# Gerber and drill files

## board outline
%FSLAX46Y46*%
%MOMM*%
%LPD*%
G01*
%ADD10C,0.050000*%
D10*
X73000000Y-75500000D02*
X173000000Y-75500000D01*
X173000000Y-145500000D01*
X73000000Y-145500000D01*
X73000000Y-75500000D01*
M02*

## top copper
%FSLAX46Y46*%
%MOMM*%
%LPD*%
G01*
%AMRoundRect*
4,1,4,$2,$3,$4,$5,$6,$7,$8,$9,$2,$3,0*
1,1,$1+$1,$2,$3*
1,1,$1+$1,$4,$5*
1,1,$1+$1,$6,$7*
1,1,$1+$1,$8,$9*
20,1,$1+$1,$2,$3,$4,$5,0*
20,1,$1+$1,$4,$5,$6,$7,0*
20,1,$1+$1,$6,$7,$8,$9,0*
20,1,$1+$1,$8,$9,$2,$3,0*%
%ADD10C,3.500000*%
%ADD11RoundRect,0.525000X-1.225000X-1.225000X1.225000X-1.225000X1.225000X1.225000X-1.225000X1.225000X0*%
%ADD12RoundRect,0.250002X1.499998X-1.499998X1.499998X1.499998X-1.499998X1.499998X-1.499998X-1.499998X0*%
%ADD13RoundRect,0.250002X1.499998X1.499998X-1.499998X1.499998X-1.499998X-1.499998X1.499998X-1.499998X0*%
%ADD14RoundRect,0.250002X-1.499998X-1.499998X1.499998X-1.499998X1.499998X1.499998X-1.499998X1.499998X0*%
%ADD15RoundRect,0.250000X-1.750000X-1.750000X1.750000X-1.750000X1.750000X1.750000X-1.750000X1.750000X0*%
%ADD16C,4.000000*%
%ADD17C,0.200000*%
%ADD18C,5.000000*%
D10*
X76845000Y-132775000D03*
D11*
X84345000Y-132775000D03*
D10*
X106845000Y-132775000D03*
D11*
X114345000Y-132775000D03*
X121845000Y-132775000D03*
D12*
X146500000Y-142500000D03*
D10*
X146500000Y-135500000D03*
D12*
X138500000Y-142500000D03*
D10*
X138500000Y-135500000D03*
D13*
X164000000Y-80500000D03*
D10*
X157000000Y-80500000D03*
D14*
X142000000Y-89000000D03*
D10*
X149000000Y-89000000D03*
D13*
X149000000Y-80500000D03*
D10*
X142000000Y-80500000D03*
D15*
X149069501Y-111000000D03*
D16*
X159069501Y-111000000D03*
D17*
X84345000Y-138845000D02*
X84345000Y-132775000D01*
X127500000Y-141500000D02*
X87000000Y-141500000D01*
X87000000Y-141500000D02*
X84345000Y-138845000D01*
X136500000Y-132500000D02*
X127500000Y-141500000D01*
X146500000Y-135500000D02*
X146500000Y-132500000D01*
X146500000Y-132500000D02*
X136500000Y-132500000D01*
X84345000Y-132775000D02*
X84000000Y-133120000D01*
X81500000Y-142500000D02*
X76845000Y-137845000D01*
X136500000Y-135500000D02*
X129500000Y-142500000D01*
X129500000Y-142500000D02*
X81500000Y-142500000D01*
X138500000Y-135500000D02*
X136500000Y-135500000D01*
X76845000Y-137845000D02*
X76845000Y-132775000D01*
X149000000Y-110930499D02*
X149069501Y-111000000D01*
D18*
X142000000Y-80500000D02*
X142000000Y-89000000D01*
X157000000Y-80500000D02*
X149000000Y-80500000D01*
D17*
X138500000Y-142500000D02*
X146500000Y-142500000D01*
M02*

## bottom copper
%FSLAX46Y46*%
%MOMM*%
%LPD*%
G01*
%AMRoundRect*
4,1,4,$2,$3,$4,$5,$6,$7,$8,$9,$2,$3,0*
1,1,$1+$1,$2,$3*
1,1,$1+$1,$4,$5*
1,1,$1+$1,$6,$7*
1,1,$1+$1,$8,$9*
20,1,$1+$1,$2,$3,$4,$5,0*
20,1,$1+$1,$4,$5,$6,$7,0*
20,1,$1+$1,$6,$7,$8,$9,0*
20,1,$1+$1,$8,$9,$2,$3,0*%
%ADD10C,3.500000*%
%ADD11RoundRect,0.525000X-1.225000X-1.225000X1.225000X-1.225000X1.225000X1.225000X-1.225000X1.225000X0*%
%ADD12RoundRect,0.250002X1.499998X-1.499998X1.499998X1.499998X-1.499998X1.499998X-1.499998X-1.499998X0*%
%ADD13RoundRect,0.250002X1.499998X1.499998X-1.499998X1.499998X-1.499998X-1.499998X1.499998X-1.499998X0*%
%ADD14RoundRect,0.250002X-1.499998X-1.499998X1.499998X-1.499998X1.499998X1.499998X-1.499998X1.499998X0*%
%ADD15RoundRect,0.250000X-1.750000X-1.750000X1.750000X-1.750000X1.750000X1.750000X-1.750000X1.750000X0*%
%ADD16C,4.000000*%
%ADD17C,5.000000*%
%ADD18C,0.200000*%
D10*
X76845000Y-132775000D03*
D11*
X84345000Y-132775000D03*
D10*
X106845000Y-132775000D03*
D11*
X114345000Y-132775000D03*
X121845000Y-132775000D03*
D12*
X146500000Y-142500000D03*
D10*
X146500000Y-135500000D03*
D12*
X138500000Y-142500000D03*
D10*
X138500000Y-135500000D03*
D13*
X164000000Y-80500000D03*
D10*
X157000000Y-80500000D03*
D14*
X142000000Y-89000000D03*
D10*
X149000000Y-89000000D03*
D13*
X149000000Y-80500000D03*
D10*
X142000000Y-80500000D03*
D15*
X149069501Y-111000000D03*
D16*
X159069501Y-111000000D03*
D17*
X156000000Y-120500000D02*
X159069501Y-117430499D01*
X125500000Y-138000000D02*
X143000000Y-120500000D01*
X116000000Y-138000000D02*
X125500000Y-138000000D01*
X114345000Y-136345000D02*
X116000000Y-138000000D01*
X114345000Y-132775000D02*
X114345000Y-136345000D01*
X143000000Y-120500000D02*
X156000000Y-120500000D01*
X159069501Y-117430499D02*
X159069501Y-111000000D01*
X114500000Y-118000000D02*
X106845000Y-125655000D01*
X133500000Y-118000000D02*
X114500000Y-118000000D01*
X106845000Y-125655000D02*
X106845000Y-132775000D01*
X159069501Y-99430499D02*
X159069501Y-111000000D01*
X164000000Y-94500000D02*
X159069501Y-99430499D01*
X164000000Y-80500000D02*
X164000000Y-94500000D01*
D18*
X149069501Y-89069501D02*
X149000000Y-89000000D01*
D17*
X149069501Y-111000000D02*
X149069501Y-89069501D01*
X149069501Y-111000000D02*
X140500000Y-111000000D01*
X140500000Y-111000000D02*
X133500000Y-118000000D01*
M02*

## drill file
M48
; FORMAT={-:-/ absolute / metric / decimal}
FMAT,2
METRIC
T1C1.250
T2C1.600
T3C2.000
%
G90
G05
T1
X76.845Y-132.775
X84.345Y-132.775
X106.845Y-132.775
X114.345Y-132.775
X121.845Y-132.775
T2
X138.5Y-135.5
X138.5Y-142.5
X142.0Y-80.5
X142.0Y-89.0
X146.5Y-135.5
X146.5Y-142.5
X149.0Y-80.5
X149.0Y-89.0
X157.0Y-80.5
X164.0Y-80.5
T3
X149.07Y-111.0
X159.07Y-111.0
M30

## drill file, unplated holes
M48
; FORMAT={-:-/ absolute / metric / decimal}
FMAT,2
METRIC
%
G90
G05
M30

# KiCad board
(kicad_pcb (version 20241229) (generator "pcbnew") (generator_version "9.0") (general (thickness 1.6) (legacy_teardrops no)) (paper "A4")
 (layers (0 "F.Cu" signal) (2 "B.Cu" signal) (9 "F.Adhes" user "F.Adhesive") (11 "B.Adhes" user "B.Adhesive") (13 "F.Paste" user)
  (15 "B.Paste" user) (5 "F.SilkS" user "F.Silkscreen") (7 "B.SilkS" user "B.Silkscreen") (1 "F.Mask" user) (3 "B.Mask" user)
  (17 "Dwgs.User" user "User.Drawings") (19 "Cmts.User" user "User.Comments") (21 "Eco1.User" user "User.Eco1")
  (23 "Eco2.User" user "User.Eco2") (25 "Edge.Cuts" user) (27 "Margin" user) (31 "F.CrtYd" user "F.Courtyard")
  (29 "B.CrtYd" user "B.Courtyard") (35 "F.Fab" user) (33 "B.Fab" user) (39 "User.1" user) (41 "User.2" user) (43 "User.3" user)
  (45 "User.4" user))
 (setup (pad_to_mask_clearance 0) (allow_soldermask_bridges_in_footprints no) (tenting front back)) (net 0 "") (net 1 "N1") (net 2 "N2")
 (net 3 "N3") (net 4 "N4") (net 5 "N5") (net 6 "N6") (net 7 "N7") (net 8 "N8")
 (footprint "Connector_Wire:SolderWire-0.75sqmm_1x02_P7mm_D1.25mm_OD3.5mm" (layer "F.Cu") (at 164 80.5 180)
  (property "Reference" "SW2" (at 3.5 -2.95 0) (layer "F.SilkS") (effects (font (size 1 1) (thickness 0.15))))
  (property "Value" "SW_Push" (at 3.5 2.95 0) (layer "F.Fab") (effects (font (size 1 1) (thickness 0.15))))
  (pad "1" thru_hole roundrect (at 0 0 180) (size 3.5 3.5) (drill 1.6) (layers "*.Cu" "*.Mask") (remove_unused_layers no)
   (roundrect_rratio 0.071429) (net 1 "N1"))
  (pad "2" thru_hole circle (at 7 0 180) (size 3.5 3.5) (drill 1.6) (layers "*.Cu" "*.Mask") (remove_unused_layers no) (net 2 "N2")))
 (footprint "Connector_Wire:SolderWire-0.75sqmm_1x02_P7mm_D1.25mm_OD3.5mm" (layer "F.Cu") (at 142 89)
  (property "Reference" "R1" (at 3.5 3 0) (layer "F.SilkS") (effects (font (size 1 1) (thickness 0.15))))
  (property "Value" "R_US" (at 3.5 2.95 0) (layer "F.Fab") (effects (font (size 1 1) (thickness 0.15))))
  (pad "1" thru_hole roundrect (at 0 0) (size 3.5 3.5) (drill 1.6) (layers "*.Cu" "*.Mask") (remove_unused_layers no)
   (roundrect_rratio 0.071429) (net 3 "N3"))
  (pad "2" thru_hole circle (at 7 0) (size 3.5 3.5) (drill 1.6) (layers "*.Cu" "*.Mask") (remove_unused_layers no) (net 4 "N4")))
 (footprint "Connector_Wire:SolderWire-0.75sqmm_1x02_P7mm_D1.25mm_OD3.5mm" (layer "F.Cu") (at 138.5 142.5 90)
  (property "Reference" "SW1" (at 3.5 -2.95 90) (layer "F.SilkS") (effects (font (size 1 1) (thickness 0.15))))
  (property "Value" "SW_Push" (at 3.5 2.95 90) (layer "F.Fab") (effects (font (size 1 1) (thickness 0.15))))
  (pad "1" thru_hole roundrect (at 0 0 90) (size 3.5 3.5) (drill 1.6) (layers "*.Cu" "*.Mask") (remove_unused_layers no)
   (roundrect_rratio 0.071429) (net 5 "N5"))
  (pad "2" thru_hole circle (at 7 0 90) (size 3.5 3.5) (drill 1.6) (layers "*.Cu" "*.Mask") (remove_unused_layers no) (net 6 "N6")))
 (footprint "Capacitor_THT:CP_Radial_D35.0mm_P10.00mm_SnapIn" (layer "F.Cu") (at 149.069501 111)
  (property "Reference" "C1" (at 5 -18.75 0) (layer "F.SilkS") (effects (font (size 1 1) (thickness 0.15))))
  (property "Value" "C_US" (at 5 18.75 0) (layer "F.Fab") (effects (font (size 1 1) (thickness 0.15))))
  (pad "1" thru_hole roundrect (at 0 0) (size 4 4) (drill 2) (layers "*.Cu" "*.Mask") (remove_unused_layers no) (roundrect_rratio 0.0625)
   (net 4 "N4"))
  (pad "2" thru_hole circle (at 10 0) (size 4 4) (drill 2) (layers "*.Cu" "*.Mask") (remove_unused_layers no) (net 1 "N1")))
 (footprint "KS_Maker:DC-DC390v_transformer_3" (layer "F.Cu") (at 104.345 102.775)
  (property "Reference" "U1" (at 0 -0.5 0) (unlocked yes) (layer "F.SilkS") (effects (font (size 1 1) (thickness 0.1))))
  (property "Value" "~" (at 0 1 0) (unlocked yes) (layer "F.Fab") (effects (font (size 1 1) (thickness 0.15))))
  (pad "1" thru_hole circle (at -27.5 30) (size 3.5 3.5) (drill 1.25) (layers "*.Cu" "*.Mask") (remove_unused_layers no) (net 6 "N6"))
  (pad "2" thru_hole roundrect (at -20 30) (size 3.5 3.5) (drill 1.25) (layers "*.Cu" "*.Mask") (remove_unused_layers no)
   (roundrect_rratio 0.15) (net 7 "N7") (thermal_bridge_angle 45))
  (pad "3" thru_hole circle (at 2.5 30) (size 3.5 3.5) (drill 1.25) (layers "*.Cu" "*.Mask") (remove_unused_layers no) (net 4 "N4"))
  (pad "4" thru_hole roundrect (at 10 30) (size 3.5 3.5) (drill 1.25) (layers "*.Cu" "*.Mask") (remove_unused_layers no)
   (roundrect_rratio 0.15) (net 1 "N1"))
  (pad "5" thru_hole roundrect (at 17.5 30) (size 3.5 3.5) (drill 1.25) (layers "*.Cu" "*.Mask") (remove_unused_layers no)
   (roundrect_rratio 0.15) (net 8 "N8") (thermal_bridge_angle 45)))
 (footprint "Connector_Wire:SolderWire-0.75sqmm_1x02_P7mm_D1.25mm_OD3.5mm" (layer "F.Cu") (at 149 80.5 180)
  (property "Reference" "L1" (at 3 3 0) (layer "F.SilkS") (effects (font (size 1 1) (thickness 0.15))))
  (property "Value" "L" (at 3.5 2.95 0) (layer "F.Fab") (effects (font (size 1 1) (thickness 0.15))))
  (pad "1" thru_hole roundrect (at 0 0 180) (size 3.5 3.5) (drill 1.6) (layers "*.Cu" "*.Mask") (remove_unused_layers no)
   (roundrect_rratio 0.071429) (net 2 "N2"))
  (pad "2" thru_hole circle (at 7 0 180) (size 3.5 3.5) (drill 1.6) (layers "*.Cu" "*.Mask") (remove_unused_layers no) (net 3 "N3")))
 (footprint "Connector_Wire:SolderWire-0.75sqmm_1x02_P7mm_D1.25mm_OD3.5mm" (layer "F.Cu") (at 146.5 142.5 90)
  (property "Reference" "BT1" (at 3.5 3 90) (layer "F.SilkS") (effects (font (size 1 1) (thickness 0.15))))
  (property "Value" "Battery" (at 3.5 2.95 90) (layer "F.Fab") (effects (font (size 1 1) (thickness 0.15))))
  (pad "1" thru_hole roundrect (at 0 0 90) (size 3.5 3.5) (drill 1.6) (layers "*.Cu" "*.Mask") (remove_unused_layers no)
   (roundrect_rratio 0.071429) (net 5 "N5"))
  (pad "2" thru_hole circle (at 7 0 90) (size 3.5 3.5) (drill 1.6) (layers "*.Cu" "*.Mask") (remove_unused_layers no) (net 7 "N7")))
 (gr_rect (start 73 75.5) (end 173 145.5) (stroke (width 0.05) (type default)) (fill no) (layer "Edge.Cuts"))
 (segment (start 146.5 132.5) (end 136.5 132.5) (width 0.2) (layer "F.Cu") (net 7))
 (segment (start 136.5 132.5) (end 127.5 141.5) (width 0.2) (layer "F.Cu") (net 7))
 (segment (start 84.345 138.845) (end 84.345 132.775) (width 0.2) (layer "F.Cu") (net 7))
 (segment (start 87 141.5) (end 84.345 138.845) (width 0.2) (layer "F.Cu") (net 7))
 (segment (start 127.5 141.5) (end 87 141.5) (width 0.2) (layer "F.Cu") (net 7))
 (segment (start 84.345 132.775) (end 84 133.12) (width 0.2) (layer "F.Cu") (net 7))
 (segment (start 146.5 135.5) (end 146.5 132.5) (width 0.2) (layer "F.Cu") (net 7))
 (segment (start 138.5 142.5) (end 146.5 142.5) (width 0.2) (layer "F.Cu") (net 5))
 (segment (start 164 80.5) (end 164 94.5) (width 5) (layer "B.Cu") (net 1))
 (segment (start 114.345 136.345) (end 116 138) (width 5) (layer "B.Cu") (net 1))
 (segment (start 164 94.5) (end 159.069501 99.430499) (width 5) (layer "B.Cu") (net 1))
 (segment (start 159.069501 99.430499) (end 159.069501 111) (width 5) (layer "B.Cu") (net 1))
 (segment (start 156 120.5) (end 159.069501 117.430499) (width 5) (layer "B.Cu") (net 1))
 (segment (start 143 120.5) (end 156 120.5) (width 5) (layer "B.Cu") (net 1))
 (segment (start 114.345 132.775) (end 114.345 136.345) (width 5) (layer "B.Cu") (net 1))
 (segment (start 116 138) (end 125.5 138) (width 5) (layer "B.Cu") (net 1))
 (segment (start 159.069501 117.430499) (end 159.069501 111) (width 5) (layer "B.Cu") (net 1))
 (segment (start 125.5 138) (end 143 120.5) (width 5) (layer "B.Cu") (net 1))
 (segment (start 149 110.930499) (end 149.069501 111) (width 0.2) (layer "F.Cu") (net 4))
 (segment (start 133.5 118) (end 114.5 118) (width 5) (layer "B.Cu") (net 4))
 (segment (start 149.069501 89.069501) (end 149 89) (width 0.2) (layer "B.Cu") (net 4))
 (segment (start 149.069501 111) (end 149.069501 89.069501) (width 5) (layer "B.Cu") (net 4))
 (segment (start 114.5 118) (end 106.845 125.655) (width 5) (layer "B.Cu") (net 4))
 (segment (start 140.5 111) (end 133.5 118) (width 5) (layer "B.Cu") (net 4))
 (segment (start 149.069501 111) (end 140.5 111) (width 5) (layer "B.Cu") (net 4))
 (segment (start 106.845 125.655) (end 106.845 132.775) (width 5) (layer "B.Cu") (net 4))
 (segment (start 142 80.5) (end 142 89) (width 5) (layer "F.Cu") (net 3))
 (segment (start 157 80.5) (end 149 80.5) (width 5) (layer "F.Cu") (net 2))
 (segment (start 81.5 142.5) (end 76.845 137.845) (width 0.2) (layer "F.Cu") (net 6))
 (segment (start 136.5 135.5) (end 129.5 142.5) (width 0.2) (layer "F.Cu") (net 6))
 (segment (start 76.845 137.845) (end 76.845 132.775) (width 0.2) (layer "F.Cu") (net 6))
 (segment (start 129.5 142.5) (end 81.5 142.5) (width 0.2) (layer "F.Cu") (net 6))
 (segment (start 138.5 135.5) (end 136.5 135.5) (width 0.2) (layer "F.Cu") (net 6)))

